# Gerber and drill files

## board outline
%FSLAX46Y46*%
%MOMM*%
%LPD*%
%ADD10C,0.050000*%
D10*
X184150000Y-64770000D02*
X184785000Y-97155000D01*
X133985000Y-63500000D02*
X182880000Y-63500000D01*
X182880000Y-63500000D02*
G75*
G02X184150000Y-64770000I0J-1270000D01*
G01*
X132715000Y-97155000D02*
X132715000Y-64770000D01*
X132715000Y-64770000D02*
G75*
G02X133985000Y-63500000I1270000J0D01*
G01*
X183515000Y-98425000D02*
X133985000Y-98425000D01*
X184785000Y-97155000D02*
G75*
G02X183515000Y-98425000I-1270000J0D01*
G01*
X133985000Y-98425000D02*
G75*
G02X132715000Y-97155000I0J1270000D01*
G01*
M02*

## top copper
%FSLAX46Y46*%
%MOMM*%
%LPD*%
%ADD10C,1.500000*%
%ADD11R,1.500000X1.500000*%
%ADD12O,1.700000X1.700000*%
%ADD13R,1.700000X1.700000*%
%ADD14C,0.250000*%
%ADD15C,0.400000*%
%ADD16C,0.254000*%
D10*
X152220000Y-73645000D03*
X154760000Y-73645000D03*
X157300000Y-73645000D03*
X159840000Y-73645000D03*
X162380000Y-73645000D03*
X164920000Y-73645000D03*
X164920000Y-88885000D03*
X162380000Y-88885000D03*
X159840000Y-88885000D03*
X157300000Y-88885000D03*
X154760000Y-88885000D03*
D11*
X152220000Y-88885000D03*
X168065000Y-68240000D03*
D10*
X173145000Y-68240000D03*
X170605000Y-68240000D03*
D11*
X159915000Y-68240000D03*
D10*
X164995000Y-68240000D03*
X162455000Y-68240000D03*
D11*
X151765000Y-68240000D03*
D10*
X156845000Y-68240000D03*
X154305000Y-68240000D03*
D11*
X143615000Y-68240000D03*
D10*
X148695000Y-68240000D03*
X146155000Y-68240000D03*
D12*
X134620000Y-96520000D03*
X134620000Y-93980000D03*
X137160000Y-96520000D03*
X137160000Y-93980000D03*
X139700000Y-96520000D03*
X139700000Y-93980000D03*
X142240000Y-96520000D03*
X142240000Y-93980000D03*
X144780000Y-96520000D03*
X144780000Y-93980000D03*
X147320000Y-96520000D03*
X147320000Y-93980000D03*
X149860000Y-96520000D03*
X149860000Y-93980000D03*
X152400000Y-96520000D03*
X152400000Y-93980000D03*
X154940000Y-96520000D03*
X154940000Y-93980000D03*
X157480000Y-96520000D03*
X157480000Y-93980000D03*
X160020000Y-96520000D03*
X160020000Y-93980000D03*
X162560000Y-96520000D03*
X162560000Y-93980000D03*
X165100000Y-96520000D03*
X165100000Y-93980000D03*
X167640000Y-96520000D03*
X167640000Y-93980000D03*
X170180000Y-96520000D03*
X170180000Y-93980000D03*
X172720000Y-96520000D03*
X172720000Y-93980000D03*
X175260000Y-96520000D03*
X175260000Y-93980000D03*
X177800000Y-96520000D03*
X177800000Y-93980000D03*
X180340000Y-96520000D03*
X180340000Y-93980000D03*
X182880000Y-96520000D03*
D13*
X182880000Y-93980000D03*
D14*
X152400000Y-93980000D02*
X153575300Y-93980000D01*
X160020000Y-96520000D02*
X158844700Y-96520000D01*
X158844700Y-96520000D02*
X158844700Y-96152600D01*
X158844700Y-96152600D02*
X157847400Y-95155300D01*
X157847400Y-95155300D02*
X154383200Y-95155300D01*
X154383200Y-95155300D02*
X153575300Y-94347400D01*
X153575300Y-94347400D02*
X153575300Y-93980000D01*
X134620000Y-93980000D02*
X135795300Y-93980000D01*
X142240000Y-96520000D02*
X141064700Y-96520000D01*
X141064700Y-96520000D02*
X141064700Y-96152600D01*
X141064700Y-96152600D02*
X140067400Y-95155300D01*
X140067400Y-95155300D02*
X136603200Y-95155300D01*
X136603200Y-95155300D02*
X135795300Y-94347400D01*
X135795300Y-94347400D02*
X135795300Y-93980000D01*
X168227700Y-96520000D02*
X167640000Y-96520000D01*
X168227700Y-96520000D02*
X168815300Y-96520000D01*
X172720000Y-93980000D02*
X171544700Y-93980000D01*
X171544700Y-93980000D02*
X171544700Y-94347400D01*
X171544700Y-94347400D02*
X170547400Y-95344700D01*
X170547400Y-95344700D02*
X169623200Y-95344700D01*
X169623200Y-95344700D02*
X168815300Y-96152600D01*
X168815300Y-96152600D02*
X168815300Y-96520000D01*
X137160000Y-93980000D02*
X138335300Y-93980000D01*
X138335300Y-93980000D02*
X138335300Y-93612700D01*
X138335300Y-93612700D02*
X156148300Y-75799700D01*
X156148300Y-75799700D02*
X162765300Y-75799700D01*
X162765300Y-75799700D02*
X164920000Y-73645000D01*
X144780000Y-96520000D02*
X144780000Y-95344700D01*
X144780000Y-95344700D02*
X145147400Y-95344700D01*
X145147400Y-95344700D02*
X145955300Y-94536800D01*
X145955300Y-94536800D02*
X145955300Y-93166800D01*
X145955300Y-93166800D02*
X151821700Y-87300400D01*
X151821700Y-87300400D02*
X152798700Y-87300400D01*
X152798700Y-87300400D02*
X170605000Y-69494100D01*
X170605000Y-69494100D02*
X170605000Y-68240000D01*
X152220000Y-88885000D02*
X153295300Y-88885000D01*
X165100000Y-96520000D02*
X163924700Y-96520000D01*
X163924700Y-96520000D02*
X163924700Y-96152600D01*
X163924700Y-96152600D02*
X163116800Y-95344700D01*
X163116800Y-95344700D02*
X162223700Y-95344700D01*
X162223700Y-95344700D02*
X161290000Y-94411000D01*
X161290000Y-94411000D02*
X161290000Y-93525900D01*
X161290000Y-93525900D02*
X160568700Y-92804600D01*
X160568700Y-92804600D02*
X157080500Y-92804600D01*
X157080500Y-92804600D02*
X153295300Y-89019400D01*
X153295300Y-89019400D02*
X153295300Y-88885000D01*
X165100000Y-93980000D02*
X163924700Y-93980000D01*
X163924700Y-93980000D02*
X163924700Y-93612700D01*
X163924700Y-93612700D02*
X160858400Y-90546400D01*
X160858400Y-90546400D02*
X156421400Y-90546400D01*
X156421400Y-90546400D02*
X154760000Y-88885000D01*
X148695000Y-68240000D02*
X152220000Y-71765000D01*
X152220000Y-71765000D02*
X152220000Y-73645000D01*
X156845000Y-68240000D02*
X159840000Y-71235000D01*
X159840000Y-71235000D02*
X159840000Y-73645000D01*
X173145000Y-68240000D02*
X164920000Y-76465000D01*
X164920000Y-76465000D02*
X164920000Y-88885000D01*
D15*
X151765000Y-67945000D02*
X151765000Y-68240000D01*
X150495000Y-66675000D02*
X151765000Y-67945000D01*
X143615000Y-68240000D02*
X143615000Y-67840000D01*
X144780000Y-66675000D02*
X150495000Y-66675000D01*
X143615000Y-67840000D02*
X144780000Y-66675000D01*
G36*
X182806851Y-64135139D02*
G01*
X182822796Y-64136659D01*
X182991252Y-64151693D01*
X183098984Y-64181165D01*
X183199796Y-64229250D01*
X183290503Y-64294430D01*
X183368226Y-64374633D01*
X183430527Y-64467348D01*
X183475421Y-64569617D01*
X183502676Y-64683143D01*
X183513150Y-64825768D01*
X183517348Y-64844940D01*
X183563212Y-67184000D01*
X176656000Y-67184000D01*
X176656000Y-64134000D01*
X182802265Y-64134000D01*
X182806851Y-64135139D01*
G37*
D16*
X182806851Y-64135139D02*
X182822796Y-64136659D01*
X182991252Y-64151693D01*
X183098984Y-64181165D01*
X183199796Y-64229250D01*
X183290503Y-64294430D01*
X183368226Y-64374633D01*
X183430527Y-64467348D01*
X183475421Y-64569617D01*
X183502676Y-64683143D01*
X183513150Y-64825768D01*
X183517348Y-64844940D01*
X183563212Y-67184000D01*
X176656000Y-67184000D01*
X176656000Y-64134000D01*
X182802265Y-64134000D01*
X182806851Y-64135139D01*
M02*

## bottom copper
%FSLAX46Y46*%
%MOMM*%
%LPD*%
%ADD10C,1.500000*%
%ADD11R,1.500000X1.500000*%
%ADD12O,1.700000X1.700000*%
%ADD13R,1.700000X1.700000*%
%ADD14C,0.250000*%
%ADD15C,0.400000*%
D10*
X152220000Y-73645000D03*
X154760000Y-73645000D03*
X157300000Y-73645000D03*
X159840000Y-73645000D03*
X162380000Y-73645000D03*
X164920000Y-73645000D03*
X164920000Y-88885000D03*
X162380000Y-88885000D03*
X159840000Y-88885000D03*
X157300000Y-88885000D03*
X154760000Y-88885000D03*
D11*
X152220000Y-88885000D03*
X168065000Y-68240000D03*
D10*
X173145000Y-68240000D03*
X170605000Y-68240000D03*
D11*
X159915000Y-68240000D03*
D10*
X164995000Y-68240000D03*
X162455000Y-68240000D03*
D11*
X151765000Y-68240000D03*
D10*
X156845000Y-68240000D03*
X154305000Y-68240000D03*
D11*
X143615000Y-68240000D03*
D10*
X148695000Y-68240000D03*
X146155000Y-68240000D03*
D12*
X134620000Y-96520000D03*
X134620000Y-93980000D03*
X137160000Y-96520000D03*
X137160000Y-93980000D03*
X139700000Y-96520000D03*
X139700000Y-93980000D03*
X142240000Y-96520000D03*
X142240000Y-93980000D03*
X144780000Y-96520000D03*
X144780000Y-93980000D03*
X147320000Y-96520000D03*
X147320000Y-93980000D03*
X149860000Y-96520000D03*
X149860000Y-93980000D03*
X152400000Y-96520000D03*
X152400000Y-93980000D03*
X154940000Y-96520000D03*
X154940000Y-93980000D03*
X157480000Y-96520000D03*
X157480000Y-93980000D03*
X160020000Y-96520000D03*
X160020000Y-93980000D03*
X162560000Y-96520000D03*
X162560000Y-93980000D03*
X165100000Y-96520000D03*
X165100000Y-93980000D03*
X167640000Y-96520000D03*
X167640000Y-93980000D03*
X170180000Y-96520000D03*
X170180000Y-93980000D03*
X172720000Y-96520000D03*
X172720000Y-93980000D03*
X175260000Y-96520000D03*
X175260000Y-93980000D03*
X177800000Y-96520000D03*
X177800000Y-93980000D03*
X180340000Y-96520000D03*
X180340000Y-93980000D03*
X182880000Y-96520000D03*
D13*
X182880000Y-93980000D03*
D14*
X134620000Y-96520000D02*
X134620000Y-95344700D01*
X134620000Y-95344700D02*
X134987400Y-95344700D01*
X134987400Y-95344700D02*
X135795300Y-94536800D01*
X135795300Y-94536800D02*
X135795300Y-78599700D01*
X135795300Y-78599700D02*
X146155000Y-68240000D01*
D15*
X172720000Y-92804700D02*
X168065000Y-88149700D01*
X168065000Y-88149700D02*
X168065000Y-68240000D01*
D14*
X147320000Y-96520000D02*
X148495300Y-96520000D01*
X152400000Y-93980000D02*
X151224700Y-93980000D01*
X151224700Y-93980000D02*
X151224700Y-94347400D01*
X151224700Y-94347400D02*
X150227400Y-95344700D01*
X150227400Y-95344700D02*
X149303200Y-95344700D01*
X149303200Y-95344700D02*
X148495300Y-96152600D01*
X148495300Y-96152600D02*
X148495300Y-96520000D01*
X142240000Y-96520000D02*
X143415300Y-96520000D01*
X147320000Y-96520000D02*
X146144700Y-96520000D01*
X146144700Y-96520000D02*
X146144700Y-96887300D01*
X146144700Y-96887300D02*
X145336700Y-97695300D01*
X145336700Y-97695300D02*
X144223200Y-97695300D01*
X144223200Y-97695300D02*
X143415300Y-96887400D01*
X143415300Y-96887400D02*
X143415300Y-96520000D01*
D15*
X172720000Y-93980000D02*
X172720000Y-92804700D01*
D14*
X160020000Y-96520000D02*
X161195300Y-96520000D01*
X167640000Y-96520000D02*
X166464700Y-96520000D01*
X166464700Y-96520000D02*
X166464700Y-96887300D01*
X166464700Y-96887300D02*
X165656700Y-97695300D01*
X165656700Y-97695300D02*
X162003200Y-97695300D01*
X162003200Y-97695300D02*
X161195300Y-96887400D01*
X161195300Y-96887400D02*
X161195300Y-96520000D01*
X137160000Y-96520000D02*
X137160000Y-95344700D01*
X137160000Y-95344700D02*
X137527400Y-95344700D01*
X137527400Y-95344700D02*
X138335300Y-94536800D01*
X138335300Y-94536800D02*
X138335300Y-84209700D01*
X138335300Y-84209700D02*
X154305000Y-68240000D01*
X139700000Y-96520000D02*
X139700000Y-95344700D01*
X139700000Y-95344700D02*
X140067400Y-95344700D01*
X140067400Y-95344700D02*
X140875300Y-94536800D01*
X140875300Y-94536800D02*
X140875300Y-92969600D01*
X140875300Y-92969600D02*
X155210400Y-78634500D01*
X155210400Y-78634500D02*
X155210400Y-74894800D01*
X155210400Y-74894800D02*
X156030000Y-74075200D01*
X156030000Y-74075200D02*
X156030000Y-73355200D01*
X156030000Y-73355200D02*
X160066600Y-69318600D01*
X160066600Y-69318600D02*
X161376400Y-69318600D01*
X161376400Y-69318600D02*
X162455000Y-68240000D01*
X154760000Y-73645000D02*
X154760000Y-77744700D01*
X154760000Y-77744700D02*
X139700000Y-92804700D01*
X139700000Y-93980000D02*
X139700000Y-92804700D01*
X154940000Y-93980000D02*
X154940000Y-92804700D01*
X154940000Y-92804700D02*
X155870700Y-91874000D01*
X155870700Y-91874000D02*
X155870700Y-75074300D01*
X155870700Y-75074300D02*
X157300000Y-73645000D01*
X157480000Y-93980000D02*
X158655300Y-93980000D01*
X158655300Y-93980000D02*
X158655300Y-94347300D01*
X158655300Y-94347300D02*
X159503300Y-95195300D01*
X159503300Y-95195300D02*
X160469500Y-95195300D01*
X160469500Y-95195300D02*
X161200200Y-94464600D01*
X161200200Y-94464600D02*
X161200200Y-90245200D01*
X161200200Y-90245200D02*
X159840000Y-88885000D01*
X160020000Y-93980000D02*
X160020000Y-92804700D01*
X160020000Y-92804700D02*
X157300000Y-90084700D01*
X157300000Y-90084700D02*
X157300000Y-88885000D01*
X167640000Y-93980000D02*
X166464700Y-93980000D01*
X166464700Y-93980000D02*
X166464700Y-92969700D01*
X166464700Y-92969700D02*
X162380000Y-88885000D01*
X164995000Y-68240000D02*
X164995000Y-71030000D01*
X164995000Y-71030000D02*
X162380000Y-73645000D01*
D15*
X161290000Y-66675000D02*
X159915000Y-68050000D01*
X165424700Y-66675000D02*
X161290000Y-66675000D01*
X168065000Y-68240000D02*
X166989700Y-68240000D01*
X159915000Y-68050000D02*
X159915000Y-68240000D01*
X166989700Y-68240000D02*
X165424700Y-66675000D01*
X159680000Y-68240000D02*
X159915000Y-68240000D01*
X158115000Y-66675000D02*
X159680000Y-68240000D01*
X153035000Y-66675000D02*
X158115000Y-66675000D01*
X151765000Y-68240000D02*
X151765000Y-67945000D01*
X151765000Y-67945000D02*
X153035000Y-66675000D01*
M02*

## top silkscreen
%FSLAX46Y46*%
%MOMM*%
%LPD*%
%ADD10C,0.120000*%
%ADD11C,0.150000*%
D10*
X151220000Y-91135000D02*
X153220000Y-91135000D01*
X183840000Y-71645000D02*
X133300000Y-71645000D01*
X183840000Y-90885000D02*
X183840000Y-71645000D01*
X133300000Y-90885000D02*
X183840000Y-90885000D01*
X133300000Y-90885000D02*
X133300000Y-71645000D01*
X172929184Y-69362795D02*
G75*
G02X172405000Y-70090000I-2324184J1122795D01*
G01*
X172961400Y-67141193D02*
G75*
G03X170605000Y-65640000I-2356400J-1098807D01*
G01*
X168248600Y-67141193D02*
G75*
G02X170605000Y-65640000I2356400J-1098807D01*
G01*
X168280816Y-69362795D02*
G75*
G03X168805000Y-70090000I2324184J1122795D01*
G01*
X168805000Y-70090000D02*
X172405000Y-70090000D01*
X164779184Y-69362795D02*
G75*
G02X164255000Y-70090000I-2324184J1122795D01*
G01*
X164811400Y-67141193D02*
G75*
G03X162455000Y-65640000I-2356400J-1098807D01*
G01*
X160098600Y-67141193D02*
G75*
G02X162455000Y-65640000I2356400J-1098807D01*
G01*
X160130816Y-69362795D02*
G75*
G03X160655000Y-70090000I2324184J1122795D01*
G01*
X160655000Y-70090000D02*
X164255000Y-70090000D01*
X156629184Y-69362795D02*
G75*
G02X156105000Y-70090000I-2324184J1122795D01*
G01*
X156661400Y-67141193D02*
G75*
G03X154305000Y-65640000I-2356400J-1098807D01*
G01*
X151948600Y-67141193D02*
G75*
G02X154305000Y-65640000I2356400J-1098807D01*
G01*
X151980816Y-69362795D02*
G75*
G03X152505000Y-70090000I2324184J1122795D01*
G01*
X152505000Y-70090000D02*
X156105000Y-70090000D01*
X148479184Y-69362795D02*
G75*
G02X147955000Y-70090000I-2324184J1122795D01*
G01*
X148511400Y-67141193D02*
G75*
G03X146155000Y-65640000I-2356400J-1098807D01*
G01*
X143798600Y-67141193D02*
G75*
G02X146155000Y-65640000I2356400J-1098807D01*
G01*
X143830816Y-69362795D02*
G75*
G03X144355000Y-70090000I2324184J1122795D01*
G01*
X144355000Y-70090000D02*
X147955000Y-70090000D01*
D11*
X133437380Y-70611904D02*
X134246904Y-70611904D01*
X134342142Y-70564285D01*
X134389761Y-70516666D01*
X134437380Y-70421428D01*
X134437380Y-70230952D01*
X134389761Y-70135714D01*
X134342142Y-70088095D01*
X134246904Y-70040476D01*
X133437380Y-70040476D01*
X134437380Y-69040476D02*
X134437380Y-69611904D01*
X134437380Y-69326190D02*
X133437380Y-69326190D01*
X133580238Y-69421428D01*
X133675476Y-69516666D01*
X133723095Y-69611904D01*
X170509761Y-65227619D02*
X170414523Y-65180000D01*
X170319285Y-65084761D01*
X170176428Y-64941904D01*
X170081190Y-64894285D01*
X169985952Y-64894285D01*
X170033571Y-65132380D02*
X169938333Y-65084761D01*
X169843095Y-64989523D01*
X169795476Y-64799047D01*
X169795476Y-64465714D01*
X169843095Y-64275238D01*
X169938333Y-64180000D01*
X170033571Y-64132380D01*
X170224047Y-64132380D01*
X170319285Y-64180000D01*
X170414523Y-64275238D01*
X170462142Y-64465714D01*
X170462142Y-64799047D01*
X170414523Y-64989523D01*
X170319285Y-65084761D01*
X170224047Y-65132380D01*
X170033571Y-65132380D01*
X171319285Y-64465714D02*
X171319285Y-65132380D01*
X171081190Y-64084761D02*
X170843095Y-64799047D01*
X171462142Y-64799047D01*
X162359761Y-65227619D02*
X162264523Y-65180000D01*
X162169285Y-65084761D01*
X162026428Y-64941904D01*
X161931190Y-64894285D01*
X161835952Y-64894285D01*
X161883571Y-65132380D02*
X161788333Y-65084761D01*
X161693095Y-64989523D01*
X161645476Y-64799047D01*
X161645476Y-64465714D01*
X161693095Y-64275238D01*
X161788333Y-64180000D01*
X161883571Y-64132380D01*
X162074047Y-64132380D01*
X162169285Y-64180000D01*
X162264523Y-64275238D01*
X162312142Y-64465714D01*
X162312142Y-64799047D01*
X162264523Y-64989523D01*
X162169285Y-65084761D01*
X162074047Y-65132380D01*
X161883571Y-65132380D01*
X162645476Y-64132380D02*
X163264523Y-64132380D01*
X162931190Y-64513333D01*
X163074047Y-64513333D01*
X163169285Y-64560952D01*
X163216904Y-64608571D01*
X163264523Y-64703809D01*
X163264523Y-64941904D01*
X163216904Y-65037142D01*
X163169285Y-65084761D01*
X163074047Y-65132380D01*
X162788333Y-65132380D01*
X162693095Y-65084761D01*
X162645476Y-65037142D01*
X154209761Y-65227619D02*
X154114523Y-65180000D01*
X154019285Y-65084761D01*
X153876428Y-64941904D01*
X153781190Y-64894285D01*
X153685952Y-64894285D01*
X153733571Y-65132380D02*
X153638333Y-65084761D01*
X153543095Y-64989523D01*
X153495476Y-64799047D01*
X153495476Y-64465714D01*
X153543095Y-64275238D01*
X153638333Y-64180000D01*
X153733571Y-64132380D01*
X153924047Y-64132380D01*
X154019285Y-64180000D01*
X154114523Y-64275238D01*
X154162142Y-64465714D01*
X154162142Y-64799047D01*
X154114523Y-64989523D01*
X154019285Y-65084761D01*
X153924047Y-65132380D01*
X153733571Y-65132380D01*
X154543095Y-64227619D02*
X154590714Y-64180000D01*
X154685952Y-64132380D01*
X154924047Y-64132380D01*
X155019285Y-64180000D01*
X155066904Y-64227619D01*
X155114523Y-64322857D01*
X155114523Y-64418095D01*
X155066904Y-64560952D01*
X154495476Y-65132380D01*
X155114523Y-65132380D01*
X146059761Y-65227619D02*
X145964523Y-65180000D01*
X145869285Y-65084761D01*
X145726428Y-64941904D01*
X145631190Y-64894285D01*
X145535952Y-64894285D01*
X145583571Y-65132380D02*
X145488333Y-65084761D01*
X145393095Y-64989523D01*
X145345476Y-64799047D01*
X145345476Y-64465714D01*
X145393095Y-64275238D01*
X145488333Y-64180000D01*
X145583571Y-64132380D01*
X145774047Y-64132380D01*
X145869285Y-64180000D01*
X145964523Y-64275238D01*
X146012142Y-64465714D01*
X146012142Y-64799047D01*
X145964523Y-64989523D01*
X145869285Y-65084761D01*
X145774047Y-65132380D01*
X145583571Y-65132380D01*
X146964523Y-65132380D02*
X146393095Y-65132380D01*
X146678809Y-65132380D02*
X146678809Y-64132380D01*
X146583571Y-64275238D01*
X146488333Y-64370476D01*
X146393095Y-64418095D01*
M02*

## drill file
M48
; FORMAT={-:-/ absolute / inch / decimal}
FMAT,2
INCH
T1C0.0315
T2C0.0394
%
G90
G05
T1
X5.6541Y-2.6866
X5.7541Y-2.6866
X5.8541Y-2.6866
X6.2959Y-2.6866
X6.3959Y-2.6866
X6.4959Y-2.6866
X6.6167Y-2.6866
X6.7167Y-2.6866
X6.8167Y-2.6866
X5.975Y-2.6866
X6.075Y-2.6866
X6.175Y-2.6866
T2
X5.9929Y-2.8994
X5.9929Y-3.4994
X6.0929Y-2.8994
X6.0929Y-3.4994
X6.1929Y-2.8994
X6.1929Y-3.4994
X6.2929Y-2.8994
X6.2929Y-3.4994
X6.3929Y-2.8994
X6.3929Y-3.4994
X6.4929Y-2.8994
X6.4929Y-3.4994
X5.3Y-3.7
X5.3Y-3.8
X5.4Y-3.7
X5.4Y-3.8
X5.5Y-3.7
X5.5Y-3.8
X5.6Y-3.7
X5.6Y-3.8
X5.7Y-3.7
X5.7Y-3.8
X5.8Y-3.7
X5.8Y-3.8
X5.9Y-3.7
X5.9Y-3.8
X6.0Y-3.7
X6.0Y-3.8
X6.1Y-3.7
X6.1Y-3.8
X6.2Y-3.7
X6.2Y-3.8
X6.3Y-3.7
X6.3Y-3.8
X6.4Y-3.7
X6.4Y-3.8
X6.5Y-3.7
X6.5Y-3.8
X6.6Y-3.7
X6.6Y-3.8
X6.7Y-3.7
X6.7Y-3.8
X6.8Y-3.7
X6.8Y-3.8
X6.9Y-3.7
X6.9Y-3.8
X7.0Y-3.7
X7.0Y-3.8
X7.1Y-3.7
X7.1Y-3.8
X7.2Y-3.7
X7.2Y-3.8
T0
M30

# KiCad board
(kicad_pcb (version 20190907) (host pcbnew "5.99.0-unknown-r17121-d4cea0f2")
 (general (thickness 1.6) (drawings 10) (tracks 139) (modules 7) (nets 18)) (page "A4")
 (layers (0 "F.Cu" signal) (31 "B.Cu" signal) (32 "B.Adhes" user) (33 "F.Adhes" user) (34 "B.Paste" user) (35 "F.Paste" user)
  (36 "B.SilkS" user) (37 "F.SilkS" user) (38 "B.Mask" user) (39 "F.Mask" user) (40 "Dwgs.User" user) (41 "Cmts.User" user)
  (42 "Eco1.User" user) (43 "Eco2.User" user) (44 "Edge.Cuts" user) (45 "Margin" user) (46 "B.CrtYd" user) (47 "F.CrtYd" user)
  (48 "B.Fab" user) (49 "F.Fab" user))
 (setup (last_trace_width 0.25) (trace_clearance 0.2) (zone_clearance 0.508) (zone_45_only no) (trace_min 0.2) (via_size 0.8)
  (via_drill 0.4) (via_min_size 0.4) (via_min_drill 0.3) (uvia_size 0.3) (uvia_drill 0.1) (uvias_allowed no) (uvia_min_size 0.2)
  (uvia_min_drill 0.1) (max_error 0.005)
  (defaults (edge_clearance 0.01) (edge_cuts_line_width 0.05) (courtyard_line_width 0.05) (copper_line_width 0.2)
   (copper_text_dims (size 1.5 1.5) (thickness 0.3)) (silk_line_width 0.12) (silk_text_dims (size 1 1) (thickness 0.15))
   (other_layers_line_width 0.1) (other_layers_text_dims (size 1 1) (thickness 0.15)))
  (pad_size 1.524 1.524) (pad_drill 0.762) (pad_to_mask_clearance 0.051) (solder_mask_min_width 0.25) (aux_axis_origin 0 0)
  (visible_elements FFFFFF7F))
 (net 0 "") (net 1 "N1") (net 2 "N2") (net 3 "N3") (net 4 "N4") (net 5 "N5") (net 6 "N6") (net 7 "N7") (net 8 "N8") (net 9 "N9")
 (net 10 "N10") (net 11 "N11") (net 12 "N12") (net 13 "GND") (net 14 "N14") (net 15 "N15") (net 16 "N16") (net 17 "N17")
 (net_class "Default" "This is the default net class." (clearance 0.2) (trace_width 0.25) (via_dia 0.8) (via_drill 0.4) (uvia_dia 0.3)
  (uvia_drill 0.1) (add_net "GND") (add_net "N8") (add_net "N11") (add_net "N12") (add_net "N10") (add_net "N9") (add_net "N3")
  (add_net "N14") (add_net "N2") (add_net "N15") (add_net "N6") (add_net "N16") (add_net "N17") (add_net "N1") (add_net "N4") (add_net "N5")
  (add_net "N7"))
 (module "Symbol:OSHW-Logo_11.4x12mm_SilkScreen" (layer "B.Cu") (at 173.99 81.28 180)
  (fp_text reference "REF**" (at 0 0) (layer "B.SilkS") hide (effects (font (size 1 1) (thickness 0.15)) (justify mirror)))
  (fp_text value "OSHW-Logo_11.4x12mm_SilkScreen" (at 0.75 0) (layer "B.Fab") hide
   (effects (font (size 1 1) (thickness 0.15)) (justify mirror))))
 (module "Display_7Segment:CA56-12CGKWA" (layer "F.Cu") (at 152.22 88.885 90)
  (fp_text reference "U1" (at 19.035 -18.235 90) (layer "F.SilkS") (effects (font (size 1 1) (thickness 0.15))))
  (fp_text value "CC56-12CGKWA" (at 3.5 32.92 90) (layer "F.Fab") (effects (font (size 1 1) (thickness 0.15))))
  (fp_line (start -2.25 -1) (end -2.25 1) (layer "F.SilkS") (width 0.12))
  (fp_line (start 17.24 31.62) (end 17.24 -18.92) (layer "F.SilkS") (width 0.12))
  (fp_line (start -2 31.62) (end 17.24 31.62) (layer "F.SilkS") (width 0.12))
  (fp_line (start -2 -18.92) (end -2 31.62) (layer "F.SilkS") (width 0.12))
  (fp_line (start -2 -18.92) (end 17.24 -18.92) (layer "F.SilkS") (width 0.12))
  (pad "12" thru_hole circle (at 15.24 0 90) (size 1.5 1.5) (drill 1) (layers *.Cu *.Mask) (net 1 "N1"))
  (pad "11" thru_hole circle (at 15.24 2.54 90) (size 1.5 1.5) (drill 1) (layers *.Cu *.Mask) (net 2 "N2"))
  (pad "10" thru_hole circle (at 15.24 5.08 90) (size 1.5 1.5) (drill 1) (layers *.Cu *.Mask) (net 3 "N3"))
  (pad "9" thru_hole circle (at 15.24 7.62 90) (size 1.5 1.5) (drill 1) (layers *.Cu *.Mask) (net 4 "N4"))
  (pad "8" thru_hole circle (at 15.24 10.16 90) (size 1.5 1.5) (drill 1) (layers *.Cu *.Mask) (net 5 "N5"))
  (pad "7" thru_hole circle (at 15.24 12.7 90) (size 1.5 1.5) (drill 1) (layers *.Cu *.Mask) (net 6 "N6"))
  (pad "6" thru_hole circle (at 0 12.7 90) (size 1.5 1.5) (drill 1) (layers *.Cu *.Mask) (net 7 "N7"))
  (pad "5" thru_hole circle (at 0 10.16 90) (size 1.5 1.5) (drill 1) (layers *.Cu *.Mask) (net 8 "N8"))
  (pad "4" thru_hole circle (at 0 7.62 90) (size 1.5 1.5) (drill 1) (layers *.Cu *.Mask) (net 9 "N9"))
  (pad "3" thru_hole circle (at 0 5.08 90) (size 1.5 1.5) (drill 1) (layers *.Cu *.Mask) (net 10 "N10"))
  (pad "2" thru_hole circle (at 0 2.54 90) (size 1.5 1.5) (drill 1) (layers *.Cu *.Mask) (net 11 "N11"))
  (pad "1" thru_hole rect (at 0 0 90) (size 1.5 1.5) (drill 1) (layers *.Cu *.Mask) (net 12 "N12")))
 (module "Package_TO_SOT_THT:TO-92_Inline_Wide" (layer "F.Cu") (at 168.065 68.24)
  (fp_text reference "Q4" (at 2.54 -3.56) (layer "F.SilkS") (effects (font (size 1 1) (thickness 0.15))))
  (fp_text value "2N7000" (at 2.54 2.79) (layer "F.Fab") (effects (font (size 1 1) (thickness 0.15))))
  (fp_arc (start 2.54 0) (end 4.34 1.85) (angle -20) (layer "F.SilkS") (width 0.12))
  (fp_arc (start 2.54 0) (end 2.54 -2.6) (angle 65) (layer "F.SilkS") (width 0.12))
  (fp_arc (start 2.54 0) (end 2.54 -2.6) (angle -65) (layer "F.SilkS") (width 0.12))
  (fp_arc (start 2.54 0) (end 0.74 1.85) (angle 20) (layer "F.SilkS") (width 0.12))
  (fp_line (start 0.74 1.85) (end 4.34 1.85) (layer "F.SilkS") (width 0.12))
  (pad "1" thru_hole rect (at 0 0 90) (size 1.5 1.5) (drill 0.8) (layers *.Cu *.Mask) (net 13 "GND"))
  (pad "3" thru_hole circle (at 5.08 0 90) (size 1.5 1.5) (drill 0.8) (layers *.Cu *.Mask) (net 7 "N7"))
  (pad "2" thru_hole circle (at 2.54 0 90) (size 1.5 1.5) (drill 0.8) (layers *.Cu *.Mask) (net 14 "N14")))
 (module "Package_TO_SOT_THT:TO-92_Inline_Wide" (layer "F.Cu") (at 159.915 68.24)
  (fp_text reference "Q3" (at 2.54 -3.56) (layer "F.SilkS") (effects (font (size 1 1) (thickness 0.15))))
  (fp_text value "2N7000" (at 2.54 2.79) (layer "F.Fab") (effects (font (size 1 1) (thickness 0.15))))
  (fp_arc (start 2.54 0) (end 4.34 1.85) (angle -20) (layer "F.SilkS") (width 0.12))
  (fp_arc (start 2.54 0) (end 2.54 -2.6) (angle 65) (layer "F.SilkS") (width 0.12))
  (fp_arc (start 2.54 0) (end 2.54 -2.6) (angle -65) (layer "F.SilkS") (width 0.12))
  (fp_arc (start 2.54 0) (end 0.74 1.85) (angle 20) (layer "F.SilkS") (width 0.12))
  (fp_line (start 0.74 1.85) (end 4.34 1.85) (layer "F.SilkS") (width 0.12))
  (pad "1" thru_hole rect (at 0 0 90) (size 1.5 1.5) (drill 0.8) (layers *.Cu *.Mask) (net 13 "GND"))
  (pad "3" thru_hole circle (at 5.08 0 90) (size 1.5 1.5) (drill 0.8) (layers *.Cu *.Mask) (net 5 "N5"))
  (pad "2" thru_hole circle (at 2.54 0 90) (size 1.5 1.5) (drill 0.8) (layers *.Cu *.Mask) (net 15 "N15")))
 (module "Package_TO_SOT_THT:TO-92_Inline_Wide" (layer "F.Cu") (at 151.765 68.24)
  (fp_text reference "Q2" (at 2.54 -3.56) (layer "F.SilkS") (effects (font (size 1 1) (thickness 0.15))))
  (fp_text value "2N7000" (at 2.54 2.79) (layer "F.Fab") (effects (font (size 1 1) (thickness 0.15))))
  (fp_arc (start 2.54 0) (end 4.34 1.85) (angle -20) (layer "F.SilkS") (width 0.12))
  (fp_arc (start 2.54 0) (end 2.54 -2.6) (angle 65) (layer "F.SilkS") (width 0.12))
  (fp_arc (start 2.54 0) (end 2.54 -2.6) (angle -65) (layer "F.SilkS") (width 0.12))
  (fp_arc (start 2.54 0) (end 0.74 1.85) (angle 20) (layer "F.SilkS") (width 0.12))
  (fp_line (start 0.74 1.85) (end 4.34 1.85) (layer "F.SilkS") (width 0.12))
  (pad "1" thru_hole rect (at 0 0 90) (size 1.5 1.5) (drill 0.8) (layers *.Cu *.Mask) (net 13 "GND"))
  (pad "3" thru_hole circle (at 5.08 0 90) (size 1.5 1.5) (drill 0.8) (layers *.Cu *.Mask) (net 4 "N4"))
  (pad "2" thru_hole circle (at 2.54 0 90) (size 1.5 1.5) (drill 0.8) (layers *.Cu *.Mask) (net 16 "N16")))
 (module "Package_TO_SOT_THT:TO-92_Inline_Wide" (layer "F.Cu") (at 143.615 68.24)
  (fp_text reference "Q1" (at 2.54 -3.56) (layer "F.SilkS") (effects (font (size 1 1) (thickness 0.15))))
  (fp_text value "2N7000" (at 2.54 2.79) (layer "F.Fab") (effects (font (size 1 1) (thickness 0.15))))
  (fp_arc (start 2.54 0) (end 4.34 1.85) (angle -20) (layer "F.SilkS") (width 0.12))
  (fp_arc (start 2.54 0) (end 2.54 -2.6) (angle 65) (layer "F.SilkS") (width 0.12))
  (fp_arc (start 2.54 0) (end 2.54 -2.6) (angle -65) (layer "F.SilkS") (width 0.12))
  (fp_arc (start 2.54 0) (end 0.74 1.85) (angle 20) (layer "F.SilkS") (width 0.12))
  (fp_line (start 0.74 1.85) (end 4.34 1.85) (layer "F.SilkS") (width 0.12))
  (pad "1" thru_hole rect (at 0 0 90) (size 1.5 1.5) (drill 0.8) (layers *.Cu *.Mask) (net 13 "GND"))
  (pad "3" thru_hole circle (at 5.08 0 90) (size 1.5 1.5) (drill 0.8) (layers *.Cu *.Mask) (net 1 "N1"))
  (pad "2" thru_hole circle (at 2.54 0 90) (size 1.5 1.5) (drill 0.8) (layers *.Cu *.Mask) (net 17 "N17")))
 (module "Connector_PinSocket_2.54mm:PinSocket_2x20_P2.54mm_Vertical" (layer "B.Cu") (at 182.88 93.98 90)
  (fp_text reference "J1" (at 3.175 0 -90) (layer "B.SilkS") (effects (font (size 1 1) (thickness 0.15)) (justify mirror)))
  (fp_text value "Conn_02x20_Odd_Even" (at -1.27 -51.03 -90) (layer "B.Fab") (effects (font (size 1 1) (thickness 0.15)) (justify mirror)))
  (pad "40" thru_hole oval (at -2.54 -48.26 90) (size 1.7 1.7) (drill 1) (layers *.Cu *.Mask) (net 17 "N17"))
  (pad "39" thru_hole oval (at 0 -48.26 90) (size 1.7 1.7) (drill 1) (layers *.Cu *.Mask) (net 13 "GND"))
  (pad "38" thru_hole oval (at -2.54 -45.72 90) (size 1.7 1.7) (drill 1) (layers *.Cu *.Mask) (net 16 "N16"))
  (pad "37" thru_hole oval (at 0 -45.72 90) (size 1.7 1.7) (drill 1) (layers *.Cu *.Mask) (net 6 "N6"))
  (pad "36" thru_hole oval (at -2.54 -43.18 90) (size 1.7 1.7) (drill 1) (layers *.Cu *.Mask) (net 15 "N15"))
  (pad "35" thru_hole oval (at 0 -43.18 90) (size 1.7 1.7) (drill 1) (layers *.Cu *.Mask) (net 2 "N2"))
  (pad "34" thru_hole oval (at -2.54 -40.64 90) (size 1.7 1.7) (drill 1) (layers *.Cu *.Mask) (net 13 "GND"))
  (pad "33" thru_hole oval (at 0 -40.64 90) (size 1.7 1.7) (drill 1) (layers *.Cu *.Mask))
  (pad "32" thru_hole oval (at -2.54 -38.1 90) (size 1.7 1.7) (drill 1) (layers *.Cu *.Mask) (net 14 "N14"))
  (pad "31" thru_hole oval (at 0 -38.1 90) (size 1.7 1.7) (drill 1) (layers *.Cu *.Mask))
  (pad "30" thru_hole oval (at -2.54 -35.56 90) (size 1.7 1.7) (drill 1) (layers *.Cu *.Mask) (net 13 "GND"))
  (pad "29" thru_hole oval (at 0 -35.56 90) (size 1.7 1.7) (drill 1) (layers *.Cu *.Mask))
  (pad "28" thru_hole oval (at -2.54 -33.02 90) (size 1.7 1.7) (drill 1) (layers *.Cu *.Mask))
  (pad "27" thru_hole oval (at 0 -33.02 90) (size 1.7 1.7) (drill 1) (layers *.Cu *.Mask))
  (pad "26" thru_hole oval (at -2.54 -30.48 90) (size 1.7 1.7) (drill 1) (layers *.Cu *.Mask))
  (pad "25" thru_hole oval (at 0 -30.48 90) (size 1.7 1.7) (drill 1) (layers *.Cu *.Mask) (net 13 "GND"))
  (pad "24" thru_hole oval (at -2.54 -27.94 90) (size 1.7 1.7) (drill 1) (layers *.Cu *.Mask))
  (pad "23" thru_hole oval (at 0 -27.94 90) (size 1.7 1.7) (drill 1) (layers *.Cu *.Mask) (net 3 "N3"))
  (pad "22" thru_hole oval (at -2.54 -25.4 90) (size 1.7 1.7) (drill 1) (layers *.Cu *.Mask))
  (pad "21" thru_hole oval (at 0 -25.4 90) (size 1.7 1.7) (drill 1) (layers *.Cu *.Mask) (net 9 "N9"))
  (pad "20" thru_hole oval (at -2.54 -22.86 90) (size 1.7 1.7) (drill 1) (layers *.Cu *.Mask) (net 13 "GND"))
  (pad "19" thru_hole oval (at 0 -22.86 90) (size 1.7 1.7) (drill 1) (layers *.Cu *.Mask) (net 10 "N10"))
  (pad "18" thru_hole oval (at -2.54 -20.32 90) (size 1.7 1.7) (drill 1) (layers *.Cu *.Mask))
  (pad "17" thru_hole oval (at 0 -20.32 90) (size 1.7 1.7) (drill 1) (layers *.Cu *.Mask))
  (pad "16" thru_hole oval (at -2.54 -17.78 90) (size 1.7 1.7) (drill 1) (layers *.Cu *.Mask) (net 12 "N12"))
  (pad "15" thru_hole oval (at 0 -17.78 90) (size 1.7 1.7) (drill 1) (layers *.Cu *.Mask) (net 11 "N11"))
  (pad "14" thru_hole oval (at -2.54 -15.24 90) (size 1.7 1.7) (drill 1) (layers *.Cu *.Mask) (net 13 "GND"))
  (pad "13" thru_hole oval (at 0 -15.24 90) (size 1.7 1.7) (drill 1) (layers *.Cu *.Mask) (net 8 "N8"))
  (pad "12" thru_hole oval (at -2.54 -12.7 90) (size 1.7 1.7) (drill 1) (layers *.Cu *.Mask))
  (pad "11" thru_hole oval (at 0 -12.7 90) (size 1.7 1.7) (drill 1) (layers *.Cu *.Mask))
  (pad "10" thru_hole oval (at -2.54 -10.16 90) (size 1.7 1.7) (drill 1) (layers *.Cu *.Mask))
  (pad "9" thru_hole oval (at 0 -10.16 90) (size 1.7 1.7) (drill 1) (layers *.Cu *.Mask) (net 13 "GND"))
  (pad "8" thru_hole oval (at -2.54 -7.62 90) (size 1.7 1.7) (drill 1) (layers *.Cu *.Mask))
  (pad "7" thru_hole oval (at 0 -7.62 90) (size 1.7 1.7) (drill 1) (layers *.Cu *.Mask))
  (pad "6" thru_hole oval (at -2.54 -5.08 90) (size 1.7 1.7) (drill 1) (layers *.Cu *.Mask))
  (pad "5" thru_hole oval (at 0 -5.08 90) (size 1.7 1.7) (drill 1) (layers *.Cu *.Mask))
  (pad "4" thru_hole oval (at -2.54 -2.54 90) (size 1.7 1.7) (drill 1) (layers *.Cu *.Mask))
  (pad "3" thru_hole oval (at 0 -2.54 90) (size 1.7 1.7) (drill 1) (layers *.Cu *.Mask))
  (pad "2" thru_hole oval (at -2.54 0 90) (size 1.7 1.7) (drill 1) (layers *.Cu *.Mask))
  (pad "1" thru_hole rect (at 0 0 90) (size 1.7 1.7) (drill 1) (layers *.Cu *.Mask)))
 (gr_line (start 184.15 64.77) (end 184.785 97.155) (layer "Edge.Cuts") (width 0.05))
 (gr_line (start 133.985 63.5) (end 182.88 63.5) (layer "Edge.Cuts") (width 0.05))
 (gr_arc (start 182.88 64.77) (end 184.15 64.77) (angle -90) (layer "Edge.Cuts") (width 0.05))
 (gr_line (start 132.715 97.155) (end 132.715 64.77) (layer "Edge.Cuts") (width 0.05))
 (gr_arc (start 133.985 64.77) (end 133.985 63.5) (angle -90) (layer "Edge.Cuts") (width 0.05))
 (gr_line (start 183.515 98.425) (end 133.985 98.425) (layer "Edge.Cuts") (width 0.05))
 (gr_arc (start 183.515 97.155) (end 183.515 98.425) (angle -90) (layer "Edge.Cuts") (width 0.05))
 (gr_arc (start 133.985 97.155) (end 132.715 97.155) (angle -90) (layer "Edge.Cuts") (width 0.05))
 (segment (start 134.62 96.52) (end 134.62 95.3447) (width 0.25) (layer "B.Cu") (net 17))
 (segment (start 134.62 95.3447) (end 134.9874 95.3447) (width 0.25) (layer "B.Cu") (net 17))
 (segment (start 134.9874 95.3447) (end 135.7953 94.5368) (width 0.25) (layer "B.Cu") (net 17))
 (segment (start 135.7953 94.5368) (end 135.7953 78.5997) (width 0.25) (layer "B.Cu") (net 17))
 (segment (start 135.7953 78.5997) (end 146.155 68.24) (width 0.25) (layer "B.Cu") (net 17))
 (segment (start 172.72 92.8047) (end 168.065 88.1497) (width 0.4) (layer "B.Cu") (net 13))
 (segment (start 168.065 88.1497) (end 168.065 68.24) (width 0.4) (layer "B.Cu") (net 13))
 (segment (start 147.32 96.52) (end 148.4953 96.52) (width 0.25) (layer "B.Cu") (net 13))
 (segment (start 152.4 93.98) (end 151.2247 93.98) (width 0.25) (layer "B.Cu") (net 13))
 (segment (start 151.2247 93.98) (end 151.2247 94.3474) (width 0.25) (layer "B.Cu") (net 13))
 (segment (start 151.2247 94.3474) (end 150.2274 95.3447) (width 0.25) (layer "B.Cu") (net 13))
 (segment (start 150.2274 95.3447) (end 149.3032 95.3447) (width 0.25) (layer "B.Cu") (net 13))
 (segment (start 149.3032 95.3447) (end 148.4953 96.1526) (width 0.25) (layer "B.Cu") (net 13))
 (segment (start 148.4953 96.1526) (end 148.4953 96.52) (width 0.25) (layer "B.Cu") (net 13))
 (segment (start 152.4 93.98) (end 153.5753 93.98) (width 0.25) (layer "F.Cu") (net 13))
 (segment (start 160.02 96.52) (end 158.8447 96.52) (width 0.25) (layer "F.Cu") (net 13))
 (segment (start 158.8447 96.52) (end 158.8447 96.1526) (width 0.25) (layer "F.Cu") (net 13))
 (segment (start 158.8447 96.1526) (end 157.8474 95.1553) (width 0.25) (layer "F.Cu") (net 13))
 (segment (start 157.8474 95.1553) (end 154.3832 95.1553) (width 0.25) (layer "F.Cu") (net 13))
 (segment (start 154.3832 95.1553) (end 153.5753 94.3474) (width 0.25) (layer "F.Cu") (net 13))
 (segment (start 153.5753 94.3474) (end 153.5753 93.98) (width 0.25) (layer "F.Cu") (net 13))
 (segment (start 134.62 93.98) (end 135.7953 93.98) (width 0.25) (layer "F.Cu") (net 13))
 (segment (start 142.24 96.52) (end 141.0647 96.52) (width 0.25) (layer "F.Cu") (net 13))
 (segment (start 141.0647 96.52) (end 141.0647 96.1526) (width 0.25) (layer "F.Cu") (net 13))
 (segment (start 141.0647 96.1526) (end 140.0674 95.1553) (width 0.25) (layer "F.Cu") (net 13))
 (segment (start 140.0674 95.1553) (end 136.6032 95.1553) (width 0.25) (layer "F.Cu") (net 13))
 (segment (start 136.6032 95.1553) (end 135.7953 94.3474) (width 0.25) (layer "F.Cu") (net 13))
 (segment (start 135.7953 94.3474) (end 135.7953 93.98) (width 0.25) (layer "F.Cu") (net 13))
 (segment (start 142.24 96.52) (end 143.4153 96.52) (width 0.25) (layer "B.Cu") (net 13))
 (segment (start 147.32 96.52) (end 146.1447 96.52) (width 0.25) (layer "B.Cu") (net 13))
 (segment (start 146.1447 96.52) (end 146.1447 96.8873) (width 0.25) (layer "B.Cu") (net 13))
 (segment (start 146.1447 96.8873) (end 145.3367 97.6953) (width 0.25) (layer "B.Cu") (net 13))
 (segment (start 145.3367 97.6953) (end 144.2232 97.6953) (width 0.25) (layer "B.Cu") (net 13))
 (segment (start 144.2232 97.6953) (end 143.4153 96.8874) (width 0.25) (layer "B.Cu") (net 13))
 (segment (start 143.4153 96.8874) (end 143.4153 96.52) (width 0.25) (layer "B.Cu") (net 13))
 (segment (start 172.72 93.98) (end 172.72 92.8047) (width 0.4) (layer "B.Cu") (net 13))
 (segment (start 160.02 96.52) (end 161.1953 96.52) (width 0.25) (layer "B.Cu") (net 13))
 (segment (start 167.64 96.52) (end 166.4647 96.52) (width 0.25) (layer "B.Cu") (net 13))
 (segment (start 166.4647 96.52) (end 166.4647 96.8873) (width 0.25) (layer "B.Cu") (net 13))
 (segment (start 166.4647 96.8873) (end 165.6567 97.6953) (width 0.25) (layer "B.Cu") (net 13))
 (segment (start 165.6567 97.6953) (end 162.0032 97.6953) (width 0.25) (layer "B.Cu") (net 13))
 (segment (start 162.0032 97.6953) (end 161.1953 96.8874) (width 0.25) (layer "B.Cu") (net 13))
 (segment (start 161.1953 96.8874) (end 161.1953 96.52) (width 0.25) (layer "B.Cu") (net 13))
 (segment (start 168.2277 96.52) (end 167.64 96.52) (width 0.25) (layer "F.Cu") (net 13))
 (segment (start 168.2277 96.52) (end 168.8153 96.52) (width 0.25) (layer "F.Cu") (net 13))
 (segment (start 172.72 93.98) (end 171.5447 93.98) (width 0.25) (layer "F.Cu") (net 13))
 (segment (start 171.5447 93.98) (end 171.5447 94.3474) (width 0.25) (layer "F.Cu") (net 13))
 (segment (start 171.5447 94.3474) (end 170.5474 95.3447) (width 0.25) (layer "F.Cu") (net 13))
 (segment (start 170.5474 95.3447) (end 169.6232 95.3447) (width 0.25) (layer "F.Cu") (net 13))
 (segment (start 169.6232 95.3447) (end 168.8153 96.1526) (width 0.25) (layer "F.Cu") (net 13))
 (segment (start 168.8153 96.1526) (end 168.8153 96.52) (width 0.25) (layer "F.Cu") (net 13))
 (segment (start 137.16 96.52) (end 137.16 95.3447) (width 0.25) (layer "B.Cu") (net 16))
 (segment (start 137.16 95.3447) (end 137.5274 95.3447) (width 0.25) (layer "B.Cu") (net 16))
 (segment (start 137.5274 95.3447) (end 138.3353 94.5368) (width 0.25) (layer "B.Cu") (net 16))
 (segment (start 138.3353 94.5368) (end 138.3353 84.2097) (width 0.25) (layer "B.Cu") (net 16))
 (segment (start 138.3353 84.2097) (end 154.305 68.24) (width 0.25) (layer "B.Cu") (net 16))
 (segment (start 137.16 93.98) (end 138.3353 93.98) (width 0.25) (layer "F.Cu") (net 6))
 (segment (start 138.3353 93.98) (end 138.3353 93.6127) (width 0.25) (layer "F.Cu") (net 6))
 (segment (start 138.3353 93.6127) (end 156.1483 75.7997) (width 0.25) (layer "F.Cu") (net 6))
 (segment (start 156.1483 75.7997) (end 162.7653 75.7997) (width 0.25) (layer "F.Cu") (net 6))
 (segment (start 162.7653 75.7997) (end 164.92 73.645) (width 0.25) (layer "F.Cu") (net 6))
 (segment (start 139.7 96.52) (end 139.7 95.3447) (width 0.25) (layer "B.Cu") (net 15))
 (segment (start 139.7 95.3447) (end 140.0674 95.3447) (width 0.25) (layer "B.Cu") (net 15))
 (segment (start 140.0674 95.3447) (end 140.8753 94.5368) (width 0.25) (layer "B.Cu") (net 15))
 (segment (start 140.8753 94.5368) (end 140.8753 92.9696) (width 0.25) (layer "B.Cu") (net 15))
 (segment (start 140.8753 92.9696) (end 155.2104 78.6345) (width 0.25) (layer "B.Cu") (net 15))
 (segment (start 155.2104 78.6345) (end 155.2104 74.8948) (width 0.25) (layer "B.Cu") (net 15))
 (segment (start 155.2104 74.8948) (end 156.03 74.0752) (width 0.25) (layer "B.Cu") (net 15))
 (segment (start 156.03 74.0752) (end 156.03 73.3552) (width 0.25) (layer "B.Cu") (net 15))
 (segment (start 156.03 73.3552) (end 160.0666 69.3186) (width 0.25) (layer "B.Cu") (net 15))
 (segment (start 160.0666 69.3186) (end 161.3764 69.3186) (width 0.25) (layer "B.Cu") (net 15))
 (segment (start 161.3764 69.3186) (end 162.455 68.24) (width 0.25) (layer "B.Cu") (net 15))
 (segment (start 154.76 73.645) (end 154.76 77.7447) (width 0.25) (layer "B.Cu") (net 2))
 (segment (start 154.76 77.7447) (end 139.7 92.8047) (width 0.25) (layer "B.Cu") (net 2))
 (segment (start 139.7 93.98) (end 139.7 92.8047) (width 0.25) (layer "B.Cu") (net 2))
 (segment (start 144.78 96.52) (end 144.78 95.3447) (width 0.25) (layer "F.Cu") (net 14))
 (segment (start 144.78 95.3447) (end 145.1474 95.3447) (width 0.25) (layer "F.Cu") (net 14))
 (segment (start 145.1474 95.3447) (end 145.9553 94.5368) (width 0.25) (layer "F.Cu") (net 14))
 (segment (start 145.9553 94.5368) (end 145.9553 93.1668) (width 0.25) (layer "F.Cu") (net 14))
 (segment (start 145.9553 93.1668) (end 151.8217 87.3004) (width 0.25) (layer "F.Cu") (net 14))
 (segment (start 151.8217 87.3004) (end 152.7987 87.3004) (width 0.25) (layer "F.Cu") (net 14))
 (segment (start 152.7987 87.3004) (end 170.605 69.4941) (width 0.25) (layer "F.Cu") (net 14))
 (segment (start 170.605 69.4941) (end 170.605 68.24) (width 0.25) (layer "F.Cu") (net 14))
 (segment (start 154.94 93.98) (end 154.94 92.8047) (width 0.25) (layer "B.Cu") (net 3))
 (segment (start 154.94 92.8047) (end 155.8707 91.874) (width 0.25) (layer "B.Cu") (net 3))
 (segment (start 155.8707 91.874) (end 155.8707 75.0743) (width 0.25) (layer "B.Cu") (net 3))
 (segment (start 155.8707 75.0743) (end 157.3 73.645) (width 0.25) (layer "B.Cu") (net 3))
 (segment (start 157.48 93.98) (end 158.6553 93.98) (width 0.25) (layer "B.Cu") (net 9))
 (segment (start 158.6553 93.98) (end 158.6553 94.3473) (width 0.25) (layer "B.Cu") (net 9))
 (segment (start 158.6553 94.3473) (end 159.5033 95.1953) (width 0.25) (layer "B.Cu") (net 9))
 (segment (start 159.5033 95.1953) (end 160.4695 95.1953) (width 0.25) (layer "B.Cu") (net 9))
 (segment (start 160.4695 95.1953) (end 161.2002 94.4646) (width 0.25) (layer "B.Cu") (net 9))
 (segment (start 161.2002 94.4646) (end 161.2002 90.2452) (width 0.25) (layer "B.Cu") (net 9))
 (segment (start 161.2002 90.2452) (end 159.84 88.885) (width 0.25) (layer "B.Cu") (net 9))
 (segment (start 160.02 93.98) (end 160.02 92.8047) (width 0.25) (layer "B.Cu") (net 10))
 (segment (start 160.02 92.8047) (end 157.3 90.0847) (width 0.25) (layer "B.Cu") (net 10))
 (segment (start 157.3 90.0847) (end 157.3 88.885) (width 0.25) (layer "B.Cu") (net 10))
 (segment (start 152.22 88.885) (end 153.2953 88.885) (width 0.25) (layer "F.Cu") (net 12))
 (segment (start 165.1 96.52) (end 163.9247 96.52) (width 0.25) (layer "F.Cu") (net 12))
 (segment (start 163.9247 96.52) (end 163.9247 96.1526) (width 0.25) (layer "F.Cu") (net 12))
 (segment (start 163.9247 96.1526) (end 163.1168 95.3447) (width 0.25) (layer "F.Cu") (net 12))
 (segment (start 163.1168 95.3447) (end 162.2237 95.3447) (width 0.25) (layer "F.Cu") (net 12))
 (segment (start 162.2237 95.3447) (end 161.29 94.411) (width 0.25) (layer "F.Cu") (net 12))
 (segment (start 161.29 94.411) (end 161.29 93.5259) (width 0.25) (layer "F.Cu") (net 12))
 (segment (start 161.29 93.5259) (end 160.5687 92.8046) (width 0.25) (layer "F.Cu") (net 12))
 (segment (start 160.5687 92.8046) (end 157.0805 92.8046) (width 0.25) (layer "F.Cu") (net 12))
 (segment (start 157.0805 92.8046) (end 153.2953 89.0194) (width 0.25) (layer "F.Cu") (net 12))
 (segment (start 153.2953 89.0194) (end 153.2953 88.885) (width 0.25) (layer "F.Cu") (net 12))
 (segment (start 165.1 93.98) (end 163.9247 93.98) (width 0.25) (layer "F.Cu") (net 11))
 (segment (start 163.9247 93.98) (end 163.9247 93.6127) (width 0.25) (layer "F.Cu") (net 11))
 (segment (start 163.9247 93.6127) (end 160.8584 90.5464) (width 0.25) (layer "F.Cu") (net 11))
 (segment (start 160.8584 90.5464) (end 156.4214 90.5464) (width 0.25) (layer "F.Cu") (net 11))
 (segment (start 156.4214 90.5464) (end 154.76 88.885) (width 0.25) (layer "F.Cu") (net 11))
 (segment (start 167.64 93.98) (end 166.4647 93.98) (width 0.25) (layer "B.Cu") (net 8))
 (segment (start 166.4647 93.98) (end 166.4647 92.9697) (width 0.25) (layer "B.Cu") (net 8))
 (segment (start 166.4647 92.9697) (end 162.38 88.885) (width 0.25) (layer "B.Cu") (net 8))
 (segment (start 148.695 68.24) (end 152.22 71.765) (width 0.25) (layer "F.Cu") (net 1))
 (segment (start 152.22 71.765) (end 152.22 73.645) (width 0.25) (layer "F.Cu") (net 1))
 (segment (start 156.845 68.24) (end 159.84 71.235) (width 0.25) (layer "F.Cu") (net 4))
 (segment (start 159.84 71.235) (end 159.84 73.645) (width 0.25) (layer "F.Cu") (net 4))
 (segment (start 164.995 68.24) (end 164.995 71.03) (width 0.25) (layer "B.Cu") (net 5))
 (segment (start 164.995 71.03) (end 162.38 73.645) (width 0.25) (layer "B.Cu") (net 5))
 (segment (start 173.145 68.24) (end 164.92 76.465) (width 0.25) (layer "F.Cu") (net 7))
 (segment (start 164.92 76.465) (end 164.92 88.885) (width 0.25) (layer "F.Cu") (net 7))
 (segment (start 161.29 66.675) (end 159.915 68.05) (width 0.4) (layer "B.Cu") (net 13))
 (segment (start 165.4247 66.675) (end 161.29 66.675) (width 0.4) (layer "B.Cu") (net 13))
 (segment (start 168.065 68.24) (end 166.9897 68.24) (width 0.4) (layer "B.Cu") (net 13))
 (segment (start 159.915 68.05) (end 159.915 68.24) (width 0.4) (layer "B.Cu") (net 13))
 (segment (start 166.9897 68.24) (end 165.4247 66.675) (width 0.4) (layer "B.Cu") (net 13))
 (segment (start 159.68 68.24) (end 159.915 68.24) (width 0.4) (layer "B.Cu") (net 13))
 (segment (start 158.115 66.675) (end 159.68 68.24) (width 0.4) (layer "B.Cu") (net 13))
 (segment (start 153.035 66.675) (end 158.115 66.675) (width 0.4) (layer "B.Cu") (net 13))
 (segment (start 151.765 68.24) (end 151.765 67.945) (width 0.4) (layer "B.Cu") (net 13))
 (segment (start 151.765 67.945) (end 153.035 66.675) (width 0.4) (layer "B.Cu") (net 13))
 (segment (start 151.765 67.945) (end 151.765 68.24) (width 0.4) (layer "F.Cu") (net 13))
 (segment (start 150.495 66.675) (end 151.765 67.945) (width 0.4) (layer "F.Cu") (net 13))
 (segment (start 143.615 68.24) (end 143.615 67.84) (width 0.4) (layer "F.Cu") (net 13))
 (segment (start 144.78 66.675) (end 150.495 66.675) (width 0.4) (layer "F.Cu") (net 13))
 (segment (start 143.615 67.84) (end 144.78 66.675) (width 0.4) (layer "F.Cu") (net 13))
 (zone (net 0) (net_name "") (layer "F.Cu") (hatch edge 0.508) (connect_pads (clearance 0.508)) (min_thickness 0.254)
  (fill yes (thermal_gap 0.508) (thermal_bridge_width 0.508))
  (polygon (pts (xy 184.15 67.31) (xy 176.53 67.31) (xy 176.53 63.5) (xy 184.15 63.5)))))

